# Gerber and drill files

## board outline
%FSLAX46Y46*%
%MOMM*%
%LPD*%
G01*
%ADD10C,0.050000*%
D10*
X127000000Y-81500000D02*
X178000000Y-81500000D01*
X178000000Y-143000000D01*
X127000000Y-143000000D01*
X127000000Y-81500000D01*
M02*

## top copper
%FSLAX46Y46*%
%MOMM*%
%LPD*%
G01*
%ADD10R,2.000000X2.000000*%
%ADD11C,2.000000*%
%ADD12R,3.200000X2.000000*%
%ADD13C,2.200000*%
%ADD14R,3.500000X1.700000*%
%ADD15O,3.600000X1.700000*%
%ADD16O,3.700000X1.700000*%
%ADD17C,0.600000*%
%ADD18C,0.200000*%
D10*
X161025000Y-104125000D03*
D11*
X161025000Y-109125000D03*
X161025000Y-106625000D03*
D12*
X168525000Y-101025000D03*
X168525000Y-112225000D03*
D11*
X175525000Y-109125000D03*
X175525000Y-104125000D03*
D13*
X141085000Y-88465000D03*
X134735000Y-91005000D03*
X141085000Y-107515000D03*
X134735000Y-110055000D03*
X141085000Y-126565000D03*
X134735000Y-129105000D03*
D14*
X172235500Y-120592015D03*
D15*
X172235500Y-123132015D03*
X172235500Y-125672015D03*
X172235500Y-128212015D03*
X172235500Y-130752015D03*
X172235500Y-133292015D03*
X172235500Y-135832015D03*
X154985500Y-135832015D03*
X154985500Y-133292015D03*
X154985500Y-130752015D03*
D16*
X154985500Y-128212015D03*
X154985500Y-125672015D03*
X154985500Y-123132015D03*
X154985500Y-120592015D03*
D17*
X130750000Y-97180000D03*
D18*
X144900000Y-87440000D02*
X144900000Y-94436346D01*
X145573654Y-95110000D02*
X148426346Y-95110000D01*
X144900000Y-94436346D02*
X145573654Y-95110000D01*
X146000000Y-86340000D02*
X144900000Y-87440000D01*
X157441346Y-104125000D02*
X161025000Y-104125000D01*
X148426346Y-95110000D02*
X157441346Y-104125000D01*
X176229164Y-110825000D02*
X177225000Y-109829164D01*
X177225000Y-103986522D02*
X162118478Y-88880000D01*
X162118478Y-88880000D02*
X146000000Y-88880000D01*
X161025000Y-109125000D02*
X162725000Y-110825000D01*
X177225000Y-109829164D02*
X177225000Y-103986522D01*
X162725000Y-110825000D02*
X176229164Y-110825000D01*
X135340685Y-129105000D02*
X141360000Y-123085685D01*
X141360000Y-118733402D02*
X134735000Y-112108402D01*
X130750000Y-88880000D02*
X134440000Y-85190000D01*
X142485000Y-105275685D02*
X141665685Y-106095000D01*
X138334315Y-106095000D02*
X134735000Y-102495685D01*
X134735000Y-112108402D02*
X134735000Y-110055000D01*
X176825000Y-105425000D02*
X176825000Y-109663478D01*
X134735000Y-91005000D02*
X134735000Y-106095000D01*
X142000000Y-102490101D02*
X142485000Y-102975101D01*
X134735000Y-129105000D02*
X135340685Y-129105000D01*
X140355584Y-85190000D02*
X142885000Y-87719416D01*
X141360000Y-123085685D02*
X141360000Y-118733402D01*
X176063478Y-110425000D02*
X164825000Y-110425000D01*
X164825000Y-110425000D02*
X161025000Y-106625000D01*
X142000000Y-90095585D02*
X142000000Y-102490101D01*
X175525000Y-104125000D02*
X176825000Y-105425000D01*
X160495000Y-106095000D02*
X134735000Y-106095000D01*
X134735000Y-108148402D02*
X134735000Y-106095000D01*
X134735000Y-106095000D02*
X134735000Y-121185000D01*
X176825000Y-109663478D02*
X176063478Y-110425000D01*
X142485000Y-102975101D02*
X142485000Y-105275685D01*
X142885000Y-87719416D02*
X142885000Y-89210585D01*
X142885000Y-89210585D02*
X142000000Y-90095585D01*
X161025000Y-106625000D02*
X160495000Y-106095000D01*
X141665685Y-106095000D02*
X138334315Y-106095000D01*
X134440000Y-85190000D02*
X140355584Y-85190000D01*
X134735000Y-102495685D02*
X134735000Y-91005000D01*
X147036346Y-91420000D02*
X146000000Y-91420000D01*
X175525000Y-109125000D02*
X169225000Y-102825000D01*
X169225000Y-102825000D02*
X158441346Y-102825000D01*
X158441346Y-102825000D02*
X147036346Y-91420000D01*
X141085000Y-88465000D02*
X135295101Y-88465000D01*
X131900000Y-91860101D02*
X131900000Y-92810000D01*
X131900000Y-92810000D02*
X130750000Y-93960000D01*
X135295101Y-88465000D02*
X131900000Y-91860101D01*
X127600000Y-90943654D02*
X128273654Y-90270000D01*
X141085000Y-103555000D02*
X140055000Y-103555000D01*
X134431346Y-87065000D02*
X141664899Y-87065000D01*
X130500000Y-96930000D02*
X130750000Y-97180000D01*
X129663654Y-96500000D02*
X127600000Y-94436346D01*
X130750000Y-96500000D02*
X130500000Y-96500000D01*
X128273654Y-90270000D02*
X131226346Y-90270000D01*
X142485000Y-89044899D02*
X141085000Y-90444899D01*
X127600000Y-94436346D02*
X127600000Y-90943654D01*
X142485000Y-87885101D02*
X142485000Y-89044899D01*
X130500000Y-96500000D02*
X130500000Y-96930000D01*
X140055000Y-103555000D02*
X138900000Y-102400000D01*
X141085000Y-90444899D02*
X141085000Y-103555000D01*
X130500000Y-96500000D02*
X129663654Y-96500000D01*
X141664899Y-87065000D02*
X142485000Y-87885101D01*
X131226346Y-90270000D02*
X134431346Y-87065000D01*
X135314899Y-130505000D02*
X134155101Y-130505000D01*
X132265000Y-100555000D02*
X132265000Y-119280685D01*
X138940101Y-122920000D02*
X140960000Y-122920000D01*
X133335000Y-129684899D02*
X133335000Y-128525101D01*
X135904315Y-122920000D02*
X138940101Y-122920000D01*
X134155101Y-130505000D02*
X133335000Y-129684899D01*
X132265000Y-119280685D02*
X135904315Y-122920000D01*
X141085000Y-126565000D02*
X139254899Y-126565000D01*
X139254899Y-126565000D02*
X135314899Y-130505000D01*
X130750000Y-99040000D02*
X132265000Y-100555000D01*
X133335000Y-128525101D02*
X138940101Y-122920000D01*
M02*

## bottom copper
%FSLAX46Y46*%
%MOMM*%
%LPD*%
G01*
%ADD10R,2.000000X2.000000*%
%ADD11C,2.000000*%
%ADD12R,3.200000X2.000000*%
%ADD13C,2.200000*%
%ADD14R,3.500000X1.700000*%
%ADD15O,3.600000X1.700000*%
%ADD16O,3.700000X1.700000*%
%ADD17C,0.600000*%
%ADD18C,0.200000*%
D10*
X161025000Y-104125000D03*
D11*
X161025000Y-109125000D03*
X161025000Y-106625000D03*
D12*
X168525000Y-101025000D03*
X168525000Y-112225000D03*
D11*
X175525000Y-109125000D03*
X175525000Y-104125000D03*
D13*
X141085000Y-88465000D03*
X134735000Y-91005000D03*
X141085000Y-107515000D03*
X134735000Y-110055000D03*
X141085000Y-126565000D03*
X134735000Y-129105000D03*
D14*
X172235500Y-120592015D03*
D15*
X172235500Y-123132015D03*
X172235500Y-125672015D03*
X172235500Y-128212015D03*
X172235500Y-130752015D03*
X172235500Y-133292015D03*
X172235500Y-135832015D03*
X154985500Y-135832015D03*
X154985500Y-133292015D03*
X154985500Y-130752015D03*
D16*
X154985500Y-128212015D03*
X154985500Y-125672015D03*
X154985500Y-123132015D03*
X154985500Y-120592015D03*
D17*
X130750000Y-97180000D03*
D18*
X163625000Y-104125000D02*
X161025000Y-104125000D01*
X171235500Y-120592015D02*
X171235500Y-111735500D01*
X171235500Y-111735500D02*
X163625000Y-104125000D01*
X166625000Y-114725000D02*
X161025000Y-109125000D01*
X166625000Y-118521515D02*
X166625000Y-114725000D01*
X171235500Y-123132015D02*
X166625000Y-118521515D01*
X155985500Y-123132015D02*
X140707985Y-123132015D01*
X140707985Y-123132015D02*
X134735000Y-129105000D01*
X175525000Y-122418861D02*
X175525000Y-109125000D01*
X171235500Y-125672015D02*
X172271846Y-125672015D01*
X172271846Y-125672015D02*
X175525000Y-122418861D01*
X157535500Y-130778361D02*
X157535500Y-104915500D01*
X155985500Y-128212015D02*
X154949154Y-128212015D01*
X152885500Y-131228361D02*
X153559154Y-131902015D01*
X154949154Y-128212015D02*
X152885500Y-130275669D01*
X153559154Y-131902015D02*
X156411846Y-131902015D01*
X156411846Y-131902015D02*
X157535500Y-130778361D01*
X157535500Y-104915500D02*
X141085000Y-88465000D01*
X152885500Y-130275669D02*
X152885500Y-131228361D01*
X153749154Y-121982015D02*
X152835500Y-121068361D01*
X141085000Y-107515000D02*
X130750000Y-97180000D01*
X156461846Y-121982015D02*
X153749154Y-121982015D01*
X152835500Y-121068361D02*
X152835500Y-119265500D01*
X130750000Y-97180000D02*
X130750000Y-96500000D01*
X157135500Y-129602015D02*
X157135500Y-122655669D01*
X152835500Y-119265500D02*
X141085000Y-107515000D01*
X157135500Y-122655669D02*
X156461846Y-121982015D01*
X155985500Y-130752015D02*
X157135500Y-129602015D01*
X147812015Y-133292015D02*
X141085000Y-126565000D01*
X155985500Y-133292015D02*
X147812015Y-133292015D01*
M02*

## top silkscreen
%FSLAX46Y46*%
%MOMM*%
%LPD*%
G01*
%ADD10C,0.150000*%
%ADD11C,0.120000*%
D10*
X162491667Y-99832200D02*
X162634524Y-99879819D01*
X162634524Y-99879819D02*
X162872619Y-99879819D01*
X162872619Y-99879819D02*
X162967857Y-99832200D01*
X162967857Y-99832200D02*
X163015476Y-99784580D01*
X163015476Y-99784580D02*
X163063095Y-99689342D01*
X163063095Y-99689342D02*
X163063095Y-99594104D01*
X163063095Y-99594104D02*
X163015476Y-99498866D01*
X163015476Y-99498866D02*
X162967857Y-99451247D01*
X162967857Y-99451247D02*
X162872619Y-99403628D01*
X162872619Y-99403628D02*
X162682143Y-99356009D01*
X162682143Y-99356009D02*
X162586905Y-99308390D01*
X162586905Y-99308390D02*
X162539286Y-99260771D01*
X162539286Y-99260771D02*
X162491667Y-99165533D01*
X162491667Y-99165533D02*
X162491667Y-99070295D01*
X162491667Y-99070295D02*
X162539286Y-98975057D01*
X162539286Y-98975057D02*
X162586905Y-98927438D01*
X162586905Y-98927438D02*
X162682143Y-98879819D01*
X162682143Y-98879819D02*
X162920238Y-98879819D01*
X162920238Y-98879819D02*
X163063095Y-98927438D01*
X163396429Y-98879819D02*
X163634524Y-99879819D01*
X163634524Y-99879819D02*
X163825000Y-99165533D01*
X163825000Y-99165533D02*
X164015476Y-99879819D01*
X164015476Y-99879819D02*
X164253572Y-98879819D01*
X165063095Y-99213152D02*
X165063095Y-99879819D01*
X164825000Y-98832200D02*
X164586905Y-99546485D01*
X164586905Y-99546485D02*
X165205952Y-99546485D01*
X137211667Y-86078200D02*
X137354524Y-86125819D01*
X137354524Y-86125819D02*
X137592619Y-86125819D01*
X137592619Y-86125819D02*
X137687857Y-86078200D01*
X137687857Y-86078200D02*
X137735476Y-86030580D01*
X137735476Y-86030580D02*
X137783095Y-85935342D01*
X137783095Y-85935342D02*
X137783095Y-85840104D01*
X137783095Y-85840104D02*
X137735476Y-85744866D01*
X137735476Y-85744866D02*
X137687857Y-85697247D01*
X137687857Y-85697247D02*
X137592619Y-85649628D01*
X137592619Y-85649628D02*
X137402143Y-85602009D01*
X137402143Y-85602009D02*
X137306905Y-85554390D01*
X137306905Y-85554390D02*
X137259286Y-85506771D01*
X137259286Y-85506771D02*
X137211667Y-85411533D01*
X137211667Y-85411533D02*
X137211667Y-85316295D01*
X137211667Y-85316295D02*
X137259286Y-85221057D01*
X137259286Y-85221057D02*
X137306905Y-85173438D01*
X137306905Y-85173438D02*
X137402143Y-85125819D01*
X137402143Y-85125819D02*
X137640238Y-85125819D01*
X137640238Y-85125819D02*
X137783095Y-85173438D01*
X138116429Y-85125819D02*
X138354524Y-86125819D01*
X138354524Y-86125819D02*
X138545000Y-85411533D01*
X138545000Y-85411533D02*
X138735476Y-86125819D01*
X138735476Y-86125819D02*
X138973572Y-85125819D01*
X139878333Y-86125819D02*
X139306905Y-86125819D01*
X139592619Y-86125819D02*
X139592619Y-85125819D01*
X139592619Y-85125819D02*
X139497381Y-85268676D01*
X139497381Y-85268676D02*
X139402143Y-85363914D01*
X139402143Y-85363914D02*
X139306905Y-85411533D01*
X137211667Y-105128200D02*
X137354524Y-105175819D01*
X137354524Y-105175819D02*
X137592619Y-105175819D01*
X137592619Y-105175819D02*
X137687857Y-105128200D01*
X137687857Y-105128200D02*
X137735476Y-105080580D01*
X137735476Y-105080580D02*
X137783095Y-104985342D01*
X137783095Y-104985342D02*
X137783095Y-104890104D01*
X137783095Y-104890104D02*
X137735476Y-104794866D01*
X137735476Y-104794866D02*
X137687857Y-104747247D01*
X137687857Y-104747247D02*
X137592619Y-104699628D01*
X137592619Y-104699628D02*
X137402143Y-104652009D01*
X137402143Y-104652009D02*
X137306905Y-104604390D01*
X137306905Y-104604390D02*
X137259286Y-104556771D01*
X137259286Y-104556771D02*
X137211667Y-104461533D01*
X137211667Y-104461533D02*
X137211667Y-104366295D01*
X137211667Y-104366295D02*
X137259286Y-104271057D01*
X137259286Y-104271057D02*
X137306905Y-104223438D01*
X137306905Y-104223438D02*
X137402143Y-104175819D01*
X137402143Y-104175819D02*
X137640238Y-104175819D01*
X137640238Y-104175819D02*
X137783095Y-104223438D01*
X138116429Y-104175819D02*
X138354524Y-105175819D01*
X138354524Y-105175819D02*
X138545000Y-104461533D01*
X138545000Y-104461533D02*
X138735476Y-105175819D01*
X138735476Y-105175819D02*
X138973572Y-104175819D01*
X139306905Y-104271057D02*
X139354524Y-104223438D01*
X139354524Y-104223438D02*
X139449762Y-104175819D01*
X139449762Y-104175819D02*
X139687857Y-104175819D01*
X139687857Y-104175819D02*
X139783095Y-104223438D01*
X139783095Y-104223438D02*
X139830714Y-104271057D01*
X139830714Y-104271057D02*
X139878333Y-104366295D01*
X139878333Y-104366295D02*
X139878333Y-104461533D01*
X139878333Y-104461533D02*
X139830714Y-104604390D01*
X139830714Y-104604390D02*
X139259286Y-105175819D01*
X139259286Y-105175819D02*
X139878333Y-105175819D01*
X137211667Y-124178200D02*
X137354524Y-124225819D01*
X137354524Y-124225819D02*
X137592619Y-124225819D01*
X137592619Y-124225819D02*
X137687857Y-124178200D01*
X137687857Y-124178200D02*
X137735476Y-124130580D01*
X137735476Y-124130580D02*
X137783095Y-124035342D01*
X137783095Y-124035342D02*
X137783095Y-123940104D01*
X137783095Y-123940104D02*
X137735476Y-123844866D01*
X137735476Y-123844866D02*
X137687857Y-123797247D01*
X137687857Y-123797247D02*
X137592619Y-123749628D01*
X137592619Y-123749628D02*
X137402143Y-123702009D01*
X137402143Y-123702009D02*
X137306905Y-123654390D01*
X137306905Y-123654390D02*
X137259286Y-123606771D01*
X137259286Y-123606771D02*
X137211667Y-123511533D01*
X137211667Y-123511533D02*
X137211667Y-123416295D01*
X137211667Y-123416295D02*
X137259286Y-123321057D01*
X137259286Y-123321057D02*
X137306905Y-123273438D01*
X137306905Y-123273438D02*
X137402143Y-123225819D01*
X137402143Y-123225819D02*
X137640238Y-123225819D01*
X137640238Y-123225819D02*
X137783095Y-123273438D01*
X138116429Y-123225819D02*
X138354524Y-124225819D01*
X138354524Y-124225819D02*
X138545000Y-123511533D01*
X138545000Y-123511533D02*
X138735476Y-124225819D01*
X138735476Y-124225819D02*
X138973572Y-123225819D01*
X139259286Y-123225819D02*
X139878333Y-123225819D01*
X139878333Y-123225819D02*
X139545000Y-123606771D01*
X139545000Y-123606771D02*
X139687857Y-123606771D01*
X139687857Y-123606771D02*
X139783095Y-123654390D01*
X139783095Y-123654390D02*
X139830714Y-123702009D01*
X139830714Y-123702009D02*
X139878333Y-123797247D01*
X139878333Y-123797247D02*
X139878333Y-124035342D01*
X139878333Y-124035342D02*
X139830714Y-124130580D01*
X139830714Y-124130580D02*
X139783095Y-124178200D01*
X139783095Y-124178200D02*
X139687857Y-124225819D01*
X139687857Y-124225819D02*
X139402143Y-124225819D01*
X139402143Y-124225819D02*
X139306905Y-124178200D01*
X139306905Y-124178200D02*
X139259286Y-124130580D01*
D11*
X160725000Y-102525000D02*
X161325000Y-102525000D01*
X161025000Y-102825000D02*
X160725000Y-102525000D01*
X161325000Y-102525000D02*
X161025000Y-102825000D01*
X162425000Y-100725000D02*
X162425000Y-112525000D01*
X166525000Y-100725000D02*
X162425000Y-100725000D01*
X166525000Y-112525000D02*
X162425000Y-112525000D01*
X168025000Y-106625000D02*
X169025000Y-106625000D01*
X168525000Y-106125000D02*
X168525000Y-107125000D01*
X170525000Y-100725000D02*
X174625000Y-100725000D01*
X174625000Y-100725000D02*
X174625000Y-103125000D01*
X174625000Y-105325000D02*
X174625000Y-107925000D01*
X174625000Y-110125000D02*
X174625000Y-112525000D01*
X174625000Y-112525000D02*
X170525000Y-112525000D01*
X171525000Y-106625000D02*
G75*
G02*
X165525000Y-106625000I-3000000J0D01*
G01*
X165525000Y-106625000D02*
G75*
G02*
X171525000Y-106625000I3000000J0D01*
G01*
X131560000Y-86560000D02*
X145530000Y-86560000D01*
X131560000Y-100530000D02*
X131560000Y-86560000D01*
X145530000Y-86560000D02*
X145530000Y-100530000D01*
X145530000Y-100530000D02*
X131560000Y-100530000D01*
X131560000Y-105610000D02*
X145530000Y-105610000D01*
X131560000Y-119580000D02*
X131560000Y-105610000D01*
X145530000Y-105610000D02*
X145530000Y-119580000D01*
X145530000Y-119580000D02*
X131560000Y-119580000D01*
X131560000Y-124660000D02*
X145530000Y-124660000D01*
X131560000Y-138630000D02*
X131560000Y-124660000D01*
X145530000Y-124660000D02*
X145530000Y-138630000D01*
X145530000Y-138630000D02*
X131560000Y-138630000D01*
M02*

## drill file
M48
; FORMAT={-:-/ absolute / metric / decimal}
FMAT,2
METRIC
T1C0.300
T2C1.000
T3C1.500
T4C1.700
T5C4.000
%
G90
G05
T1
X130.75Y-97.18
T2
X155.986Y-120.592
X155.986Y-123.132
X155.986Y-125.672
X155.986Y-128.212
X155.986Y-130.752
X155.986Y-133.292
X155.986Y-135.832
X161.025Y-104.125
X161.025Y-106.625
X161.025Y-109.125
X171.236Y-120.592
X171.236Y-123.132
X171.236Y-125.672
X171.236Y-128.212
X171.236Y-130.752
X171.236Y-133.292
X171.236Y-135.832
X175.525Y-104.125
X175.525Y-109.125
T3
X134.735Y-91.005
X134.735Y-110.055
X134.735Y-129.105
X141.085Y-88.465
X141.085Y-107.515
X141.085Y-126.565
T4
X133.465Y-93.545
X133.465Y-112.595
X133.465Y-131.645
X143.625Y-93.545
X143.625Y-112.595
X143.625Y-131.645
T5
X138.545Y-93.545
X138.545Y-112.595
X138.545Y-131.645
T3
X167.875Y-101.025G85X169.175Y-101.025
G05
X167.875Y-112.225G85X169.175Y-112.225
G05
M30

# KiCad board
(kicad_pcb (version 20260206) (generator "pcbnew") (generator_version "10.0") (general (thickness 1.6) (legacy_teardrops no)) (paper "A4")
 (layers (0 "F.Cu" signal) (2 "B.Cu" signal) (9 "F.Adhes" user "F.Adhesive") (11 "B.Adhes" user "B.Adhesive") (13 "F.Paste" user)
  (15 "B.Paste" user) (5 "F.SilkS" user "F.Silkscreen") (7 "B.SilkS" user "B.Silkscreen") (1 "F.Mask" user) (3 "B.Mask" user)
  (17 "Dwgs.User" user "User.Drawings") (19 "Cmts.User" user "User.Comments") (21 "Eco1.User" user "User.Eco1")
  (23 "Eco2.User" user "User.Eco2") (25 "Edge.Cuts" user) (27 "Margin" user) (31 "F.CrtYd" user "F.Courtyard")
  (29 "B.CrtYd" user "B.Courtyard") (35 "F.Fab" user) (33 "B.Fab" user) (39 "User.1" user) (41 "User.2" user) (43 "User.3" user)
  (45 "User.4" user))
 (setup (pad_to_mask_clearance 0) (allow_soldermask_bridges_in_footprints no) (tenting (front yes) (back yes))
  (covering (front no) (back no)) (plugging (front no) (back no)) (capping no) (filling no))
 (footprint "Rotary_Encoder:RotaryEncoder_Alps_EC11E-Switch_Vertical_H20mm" (layer "F.Cu") (at 161.025 104.125)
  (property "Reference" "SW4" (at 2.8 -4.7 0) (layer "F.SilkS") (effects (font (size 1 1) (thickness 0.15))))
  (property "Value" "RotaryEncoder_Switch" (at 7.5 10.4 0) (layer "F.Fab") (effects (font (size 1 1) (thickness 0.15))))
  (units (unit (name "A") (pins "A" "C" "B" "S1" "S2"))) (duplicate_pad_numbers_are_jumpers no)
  (fp_line (start -0.3 -1.6) (end 0.3 -1.6) (stroke (width 0.12) (type solid)) (layer "F.SilkS"))
  (fp_line (start 0 -1.3) (end -0.3 -1.6) (stroke (width 0.12) (type solid)) (layer "F.SilkS"))
  (fp_line (start 0.3 -1.6) (end 0 -1.3) (stroke (width 0.12) (type solid)) (layer "F.SilkS"))
  (fp_line (start 1.4 -3.4) (end 1.4 8.4) (stroke (width 0.12) (type solid)) (layer "F.SilkS"))
  (fp_line (start 5.5 -3.4) (end 1.4 -3.4) (stroke (width 0.12) (type solid)) (layer "F.SilkS"))
  (fp_line (start 5.5 8.4) (end 1.4 8.4) (stroke (width 0.12) (type solid)) (layer "F.SilkS"))
  (fp_line (start 7 2.5) (end 8 2.5) (stroke (width 0.12) (type solid)) (layer "F.SilkS"))
  (fp_line (start 7.5 2) (end 7.5 3) (stroke (width 0.12) (type solid)) (layer "F.SilkS"))
  (fp_line (start 9.5 -3.4) (end 13.6 -3.4) (stroke (width 0.12) (type solid)) (layer "F.SilkS"))
  (fp_line (start 13.6 -3.4) (end 13.6 -1) (stroke (width 0.12) (type solid)) (layer "F.SilkS"))
  (fp_line (start 13.6 1.2) (end 13.6 3.8) (stroke (width 0.12) (type solid)) (layer "F.SilkS"))
  (fp_line (start 13.6 6) (end 13.6 8.4) (stroke (width 0.12) (type solid)) (layer "F.SilkS"))
  (fp_line (start 13.6 8.4) (end 9.5 8.4) (stroke (width 0.12) (type solid)) (layer "F.SilkS"))
  (fp_circle (center 7.5 2.5) (end 10.5 2.5) (stroke (width 0.12) (type solid)) (fill no) (layer "F.SilkS"))
  (pad "A" thru_hole rect (at 0 0) (size 2 2) (drill 1) (layers "*.Cu" "*.Mask") (remove_unused_layers no) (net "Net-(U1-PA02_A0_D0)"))
  (pad "B" thru_hole circle (at 0 5) (size 2 2) (drill 1) (layers "*.Cu" "*.Mask") (remove_unused_layers no) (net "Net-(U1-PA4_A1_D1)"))
  (pad "C" thru_hole circle (at 0 2.5) (size 2 2) (drill 1) (layers "*.Cu" "*.Mask") (remove_unused_layers no) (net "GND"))
  (pad "MP" thru_hole rect (at 7.5 -3.1) (size 3.2 2) (drill oval 2.8 1.5) (layers "*.Cu" "*.Mask") (remove_unused_layers no))
  (pad "MP" thru_hole rect (at 7.5 8.1) (size 3.2 2) (drill oval 2.8 1.5) (layers "*.Cu" "*.Mask") (remove_unused_layers no))
  (pad "S1" thru_hole circle (at 14.5 5) (size 2 2) (drill 1) (layers "*.Cu" "*.Mask") (remove_unused_layers no) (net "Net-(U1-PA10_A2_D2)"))
  (pad "S2" thru_hole circle (at 14.5 0) (size 2 2) (drill 1) (layers "*.Cu" "*.Mask") (remove_unused_layers no) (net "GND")))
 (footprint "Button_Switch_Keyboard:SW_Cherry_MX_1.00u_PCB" (layer "F.Cu") (at 141.085 88.465)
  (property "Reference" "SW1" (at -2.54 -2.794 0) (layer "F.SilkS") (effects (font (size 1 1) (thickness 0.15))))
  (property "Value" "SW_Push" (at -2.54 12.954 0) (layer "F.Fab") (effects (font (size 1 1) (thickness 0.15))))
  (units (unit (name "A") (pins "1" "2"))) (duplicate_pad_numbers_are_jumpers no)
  (fp_line (start -9.525 -1.905) (end 4.445 -1.905) (stroke (width 0.12) (type solid)) (layer "F.SilkS"))
  (fp_line (start -9.525 12.065) (end -9.525 -1.905) (stroke (width 0.12) (type solid)) (layer "F.SilkS"))
  (fp_line (start 4.445 -1.905) (end 4.445 12.065) (stroke (width 0.12) (type solid)) (layer "F.SilkS"))
  (fp_line (start 4.445 12.065) (end -9.525 12.065) (stroke (width 0.12) (type solid)) (layer "F.SilkS"))
  (pad "" np_thru_hole circle (at -7.62 5.08) (size 1.7 1.7) (drill 1.7) (layers "*.Cu" "*.Mask"))
  (pad "" np_thru_hole circle (at -2.54 5.08) (size 4 4) (drill 4) (layers "*.Cu" "*.Mask"))
  (pad "" np_thru_hole circle (at 2.54 5.08) (size 1.7 1.7) (drill 1.7) (layers "*.Cu" "*.Mask"))
  (pad "1" thru_hole circle (at 0 0) (size 2.2 2.2) (drill 1.5) (layers "*.Cu" "*.Mask") (remove_unused_layers no)
   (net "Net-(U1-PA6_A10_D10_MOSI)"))
  (pad "2" thru_hole circle (at -6.35 2.54) (size 2.2 2.2) (drill 1.5) (layers "*.Cu" "*.Mask") (remove_unused_layers no) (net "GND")))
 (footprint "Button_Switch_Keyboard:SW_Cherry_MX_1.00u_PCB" (layer "F.Cu") (at 141.085 107.515)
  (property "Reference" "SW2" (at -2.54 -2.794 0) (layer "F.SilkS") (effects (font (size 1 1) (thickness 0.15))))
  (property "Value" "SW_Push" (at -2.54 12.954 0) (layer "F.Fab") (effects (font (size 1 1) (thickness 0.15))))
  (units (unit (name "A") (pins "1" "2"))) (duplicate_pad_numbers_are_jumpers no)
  (fp_line (start -9.525 -1.905) (end 4.445 -1.905) (stroke (width 0.12) (type solid)) (layer "F.SilkS"))
  (fp_line (start -9.525 12.065) (end -9.525 -1.905) (stroke (width 0.12) (type solid)) (layer "F.SilkS"))
  (fp_line (start 4.445 -1.905) (end 4.445 12.065) (stroke (width 0.12) (type solid)) (layer "F.SilkS"))
  (fp_line (start 4.445 12.065) (end -9.525 12.065) (stroke (width 0.12) (type solid)) (layer "F.SilkS"))
  (pad "" np_thru_hole circle (at -7.62 5.08) (size 1.7 1.7) (drill 1.7) (layers "*.Cu" "*.Mask"))
  (pad "" np_thru_hole circle (at -2.54 5.08) (size 4 4) (drill 4) (layers "*.Cu" "*.Mask"))
  (pad "" np_thru_hole circle (at 2.54 5.08) (size 1.7 1.7) (drill 1.7) (layers "*.Cu" "*.Mask"))
  (pad "1" thru_hole circle (at 0 0) (size 2.2 2.2) (drill 1.5) (layers "*.Cu" "*.Mask") (remove_unused_layers no)
   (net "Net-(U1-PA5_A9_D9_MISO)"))
  (pad "2" thru_hole circle (at -6.35 2.54) (size 2.2 2.2) (drill 1.5) (layers "*.Cu" "*.Mask") (remove_unused_layers no) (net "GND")))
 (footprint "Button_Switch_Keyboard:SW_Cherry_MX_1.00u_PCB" (layer "F.Cu") (at 141.085 126.565)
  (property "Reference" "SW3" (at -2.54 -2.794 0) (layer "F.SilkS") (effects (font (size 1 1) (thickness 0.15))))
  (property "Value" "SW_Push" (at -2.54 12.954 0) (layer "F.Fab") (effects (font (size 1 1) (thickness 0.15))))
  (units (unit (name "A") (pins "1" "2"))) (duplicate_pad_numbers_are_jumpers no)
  (fp_line (start -9.525 -1.905) (end 4.445 -1.905) (stroke (width 0.12) (type solid)) (layer "F.SilkS"))
  (fp_line (start -9.525 12.065) (end -9.525 -1.905) (stroke (width 0.12) (type solid)) (layer "F.SilkS"))
  (fp_line (start 4.445 -1.905) (end 4.445 12.065) (stroke (width 0.12) (type solid)) (layer "F.SilkS"))
  (fp_line (start 4.445 12.065) (end -9.525 12.065) (stroke (width 0.12) (type solid)) (layer "F.SilkS"))
  (pad "" np_thru_hole circle (at -7.62 5.08) (size 1.7 1.7) (drill 1.7) (layers "*.Cu" "*.Mask"))
  (pad "" np_thru_hole circle (at -2.54 5.08) (size 4 4) (drill 4) (layers "*.Cu" "*.Mask"))
  (pad "" np_thru_hole circle (at 2.54 5.08) (size 1.7 1.7) (drill 1.7) (layers "*.Cu" "*.Mask"))
  (pad "1" thru_hole circle (at 0 0) (size 2.2 2.2) (drill 1.5) (layers "*.Cu" "*.Mask") (remove_unused_layers no)
   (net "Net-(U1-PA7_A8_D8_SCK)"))
  (pad "2" thru_hole circle (at -6.35 2.54) (size 2.2 2.2) (drill 1.5) (layers "*.Cu" "*.Mask") (remove_unused_layers no) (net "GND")))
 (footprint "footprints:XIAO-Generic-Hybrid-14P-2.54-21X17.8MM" (layer "B.Cu") (at 163.6105 128.212015 180)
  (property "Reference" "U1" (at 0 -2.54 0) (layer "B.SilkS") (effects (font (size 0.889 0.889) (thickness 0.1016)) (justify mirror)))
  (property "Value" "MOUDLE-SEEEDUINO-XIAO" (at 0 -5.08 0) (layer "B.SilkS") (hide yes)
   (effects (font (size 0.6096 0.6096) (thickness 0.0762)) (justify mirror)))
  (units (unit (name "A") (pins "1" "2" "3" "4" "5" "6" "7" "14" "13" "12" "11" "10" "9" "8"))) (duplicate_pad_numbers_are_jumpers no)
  (pad "1" thru_hole rect (at -7.625 7.62 180) (size 3.5 1.7) (drill 1 (offset -1 0)) (layers "*.Cu" "*.Mask") (remove_unused_layers no)
   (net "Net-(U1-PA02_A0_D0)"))
  (pad "2" thru_hole oval (at -7.625 5.08 180) (size 3.6 1.7) (drill 1 (offset -1 0)) (layers "*.Cu" "*.Mask") (remove_unused_layers no)
   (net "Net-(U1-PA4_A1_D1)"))
  (pad "3" thru_hole oval (at -7.625 2.54 180) (size 3.6 1.7) (drill 1 (offset -1 0)) (layers "*.Cu" "*.Mask") (remove_unused_layers no)
   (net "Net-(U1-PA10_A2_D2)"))
  (pad "4" thru_hole oval (at -7.625 0 180) (size 3.6 1.7) (drill 1 (offset -1 0)) (layers "*.Cu" "*.Mask") (remove_unused_layers no)
   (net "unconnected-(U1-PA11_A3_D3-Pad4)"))
  (pad "5" thru_hole oval (at -7.625 -2.54 180) (size 3.6 1.7) (drill 1 (offset -1 0)) (layers "*.Cu" "*.Mask") (remove_unused_layers no)
   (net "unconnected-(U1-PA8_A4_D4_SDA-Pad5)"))
  (pad "6" thru_hole oval (at -7.625 -5.08) (size 3.6 1.7) (drill 1 (offset 1 0)) (layers "*.Cu" "*.Mask") (remove_unused_layers no)
   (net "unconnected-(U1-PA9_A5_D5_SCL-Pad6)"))
  (pad "7" thru_hole oval (at -7.625 -7.62 180) (size 3.6 1.7) (drill 1 (offset -1 0)) (layers "*.Cu" "*.Mask") (remove_unused_layers no)
   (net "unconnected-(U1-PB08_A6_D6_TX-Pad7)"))
  (pad "8" thru_hole oval (at 7.625 -7.62 180) (size 3.6 1.7) (drill 1 (offset 1 0)) (layers "*.Cu" "*.Mask") (remove_unused_layers no)
   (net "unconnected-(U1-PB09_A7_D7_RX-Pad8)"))
  (pad "9" thru_hole oval (at 7.625 -5.08 180) (size 3.6 1.7) (drill 1 (offset 1 0)) (layers "*.Cu" "*.Mask") (remove_unused_layers no)
   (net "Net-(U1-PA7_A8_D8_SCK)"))
  (pad "10" thru_hole oval (at 7.625 -2.54 180) (size 3.6 1.7) (drill 1 (offset 1 0)) (layers "*.Cu" "*.Mask") (remove_unused_layers no)
   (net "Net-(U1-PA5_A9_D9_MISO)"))
  (pad "11" thru_hole oval (at 7.625 0 180) (size 3.7 1.7) (drill 1 (offset 1 0)) (layers "*.Cu" "*.Mask") (remove_unused_layers no)
   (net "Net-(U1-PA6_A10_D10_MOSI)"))
  (pad "12" thru_hole oval (at 7.625 2.54 180) (size 3.7 1.7) (drill 1 (offset 1 0)) (layers "*.Cu" "*.Mask") (remove_unused_layers no)
   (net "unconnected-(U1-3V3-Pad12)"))
  (pad "13" thru_hole oval (at 7.625 5.08 180) (size 3.7 1.7) (drill 1 (offset 1 0)) (layers "*.Cu" "*.Mask") (remove_unused_layers no)
   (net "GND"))
  (pad "14" thru_hole oval (at 7.625 7.62 180) (size 3.7 1.7) (drill 1 (offset 1 0)) (layers "*.Cu" "*.Mask") (remove_unused_layers no)
   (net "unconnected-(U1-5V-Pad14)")))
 (gr_rect (start 127 81.5) (end 178 143) (stroke (width 0.05) (type solid)) (fill no) (layer "Edge.Cuts"))
 (segment (start 144.9 87.44) (end 144.9 94.436346) (width 0.2) (layer "F.Cu") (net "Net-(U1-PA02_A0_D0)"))
 (segment (start 145.573654 95.11) (end 148.426346 95.11) (width 0.2) (layer "F.Cu") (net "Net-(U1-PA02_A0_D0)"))
 (segment (start 144.9 94.436346) (end 145.573654 95.11) (width 0.2) (layer "F.Cu") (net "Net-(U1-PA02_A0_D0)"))
 (segment (start 146 86.34) (end 144.9 87.44) (width 0.2) (layer "F.Cu") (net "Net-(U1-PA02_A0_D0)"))
 (segment (start 157.441346 104.125) (end 161.025 104.125) (width 0.2) (layer "F.Cu") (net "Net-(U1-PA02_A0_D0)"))
 (segment (start 148.426346 95.11) (end 157.441346 104.125) (width 0.2) (layer "F.Cu") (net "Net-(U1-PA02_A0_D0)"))
 (segment (start 163.625 104.125) (end 161.025 104.125) (width 0.2) (layer "B.Cu") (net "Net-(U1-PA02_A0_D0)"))
 (segment (start 171.2355 120.592015) (end 171.2355 111.7355) (width 0.2) (layer "B.Cu") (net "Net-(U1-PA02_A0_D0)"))
 (segment (start 171.2355 111.7355) (end 163.625 104.125) (width 0.2) (layer "B.Cu") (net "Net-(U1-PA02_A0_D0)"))
 (segment (start 176.229164 110.825) (end 177.225 109.829164) (width 0.2) (layer "F.Cu") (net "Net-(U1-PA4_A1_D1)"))
 (segment (start 177.225 103.986522) (end 162.118478 88.88) (width 0.2) (layer "F.Cu") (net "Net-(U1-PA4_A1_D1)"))
 (segment (start 162.118478 88.88) (end 146 88.88) (width 0.2) (layer "F.Cu") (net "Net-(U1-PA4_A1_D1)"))
 (segment (start 161.025 109.125) (end 162.725 110.825) (width 0.2) (layer "F.Cu") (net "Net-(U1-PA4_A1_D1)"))
 (segment (start 177.225 109.829164) (end 177.225 103.986522) (width 0.2) (layer "F.Cu") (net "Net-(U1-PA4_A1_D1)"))
 (segment (start 162.725 110.825) (end 176.229164 110.825) (width 0.2) (layer "F.Cu") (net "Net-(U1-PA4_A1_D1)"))
 (segment (start 166.625 114.725) (end 161.025 109.125) (width 0.2) (layer "B.Cu") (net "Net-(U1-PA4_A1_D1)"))
 (segment (start 166.625 118.521515) (end 166.625 114.725) (width 0.2) (layer "B.Cu") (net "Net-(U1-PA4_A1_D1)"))
 (segment (start 171.2355 123.132015) (end 166.625 118.521515) (width 0.2) (layer "B.Cu") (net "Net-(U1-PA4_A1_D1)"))
 (segment (start 135.340685 129.105) (end 141.36 123.085685) (width 0.2) (layer "F.Cu") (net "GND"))
 (segment (start 141.36 118.733402) (end 134.735 112.108402) (width 0.2) (layer "F.Cu") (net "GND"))
 (segment (start 130.75 88.88) (end 134.44 85.19) (width 0.2) (layer "F.Cu") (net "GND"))
 (segment (start 142.485 105.275685) (end 141.665685 106.095) (width 0.2) (layer "F.Cu") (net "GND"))
 (segment (start 138.334315 106.095) (end 134.735 102.495685) (width 0.2) (layer "F.Cu") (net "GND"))
 (segment (start 134.735 112.108402) (end 134.735 110.055) (width 0.2) (layer "F.Cu") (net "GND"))
 (segment (start 176.825 105.425) (end 176.825 109.663478) (width 0.2) (layer "F.Cu") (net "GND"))
 (segment (start 134.735 91.005) (end 134.735 106.095) (width 0.2) (layer "F.Cu") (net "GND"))
 (segment (start 142 102.490101) (end 142.485 102.975101) (width 0.2) (layer "F.Cu") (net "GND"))
 (segment (start 134.735 129.105) (end 135.340685 129.105) (width 0.2) (layer "F.Cu") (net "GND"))
 (segment (start 140.355584 85.19) (end 142.885 87.719416) (width 0.2) (layer "F.Cu") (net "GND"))
 (segment (start 141.36 123.085685) (end 141.36 118.733402) (width 0.2) (layer "F.Cu") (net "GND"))
 (segment (start 176.063478 110.425) (end 164.825 110.425) (width 0.2) (layer "F.Cu") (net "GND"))
 (segment (start 164.825 110.425) (end 161.025 106.625) (width 0.2) (layer "F.Cu") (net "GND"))
 (segment (start 142 90.095585) (end 142 102.490101) (width 0.2) (layer "F.Cu") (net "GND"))
 (segment (start 175.525 104.125) (end 176.825 105.425) (width 0.2) (layer "F.Cu") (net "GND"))
 (segment (start 160.495 106.095) (end 134.735 106.095) (width 0.2) (layer "F.Cu") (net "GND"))
 (segment (start 134.735 108.148402) (end 134.735 106.095) (width 0.2) (layer "F.Cu") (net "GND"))
 (segment (start 134.735 106.095) (end 134.735 121.185) (width 0.2) (layer "F.Cu") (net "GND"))
 (segment (start 176.825 109.663478) (end 176.063478 110.425) (width 0.2) (layer "F.Cu") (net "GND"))
 (segment (start 142.485 102.975101) (end 142.485 105.275685) (width 0.2) (layer "F.Cu") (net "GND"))
 (segment (start 142.885 87.719416) (end 142.885 89.210585) (width 0.2) (layer "F.Cu") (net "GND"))
 (segment (start 142.885 89.210585) (end 142 90.095585) (width 0.2) (layer "F.Cu") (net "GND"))
 (segment (start 161.025 106.625) (end 160.495 106.095) (width 0.2) (layer "F.Cu") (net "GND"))
 (segment (start 141.665685 106.095) (end 138.334315 106.095) (width 0.2) (layer "F.Cu") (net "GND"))
 (segment (start 134.44 85.19) (end 140.355584 85.19) (width 0.2) (layer "F.Cu") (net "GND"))
 (segment (start 134.735 102.495685) (end 134.735 91.005) (width 0.2) (layer "F.Cu") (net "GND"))
 (segment (start 155.9855 123.132015) (end 140.707985 123.132015) (width 0.2) (layer "B.Cu") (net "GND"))
 (segment (start 140.707985 123.132015) (end 134.735 129.105) (width 0.2) (layer "B.Cu") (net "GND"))
 (segment (start 147.036346 91.42) (end 146 91.42) (width 0.2) (layer "F.Cu") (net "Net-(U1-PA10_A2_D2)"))
 (segment (start 175.525 109.125) (end 169.225 102.825) (width 0.2) (layer "F.Cu") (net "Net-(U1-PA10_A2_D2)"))
 (segment (start 169.225 102.825) (end 158.441346 102.825) (width 0.2) (layer "F.Cu") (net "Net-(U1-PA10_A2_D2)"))
 (segment (start 158.441346 102.825) (end 147.036346 91.42) (width 0.2) (layer "F.Cu") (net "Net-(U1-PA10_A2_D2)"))
 (segment (start 175.525 122.418861) (end 175.525 109.125) (width 0.2) (layer "B.Cu") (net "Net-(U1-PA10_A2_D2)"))
 (segment (start 171.2355 125.672015) (end 172.271846 125.672015) (width 0.2) (layer "B.Cu") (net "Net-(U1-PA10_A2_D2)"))
 (segment (start 172.271846 125.672015) (end 175.525 122.418861) (width 0.2) (layer "B.Cu") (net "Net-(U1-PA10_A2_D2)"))
 (segment (start 141.085 88.465) (end 135.295101 88.465) (width 0.2) (layer "F.Cu") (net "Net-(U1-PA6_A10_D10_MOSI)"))
 (segment (start 131.9 91.860101) (end 131.9 92.81) (width 0.2) (layer "F.Cu") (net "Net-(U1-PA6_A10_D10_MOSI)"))
 (segment (start 131.9 92.81) (end 130.75 93.96) (width 0.2) (layer "F.Cu") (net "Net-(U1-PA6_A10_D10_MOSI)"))
 (segment (start 135.295101 88.465) (end 131.9 91.860101) (width 0.2) (layer "F.Cu") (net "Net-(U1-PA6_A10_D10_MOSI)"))
 (segment (start 157.5355 130.778361) (end 157.5355 104.9155) (width 0.2) (layer "B.Cu") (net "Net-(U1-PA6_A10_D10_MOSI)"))
 (segment (start 155.9855 128.212015) (end 154.949154 128.212015) (width 0.2) (layer "B.Cu") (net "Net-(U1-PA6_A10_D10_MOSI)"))
 (segment (start 152.8855 131.228361) (end 153.559154 131.902015) (width 0.2) (layer "B.Cu") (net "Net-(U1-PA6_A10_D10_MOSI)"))
 (segment (start 154.949154 128.212015) (end 152.8855 130.275669) (width 0.2) (layer "B.Cu") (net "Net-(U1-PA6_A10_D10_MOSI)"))
 (segment (start 153.559154 131.902015) (end 156.411846 131.902015) (width 0.2) (layer "B.Cu") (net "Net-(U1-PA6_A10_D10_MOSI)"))
 (segment (start 156.411846 131.902015) (end 157.5355 130.778361) (width 0.2) (layer "B.Cu") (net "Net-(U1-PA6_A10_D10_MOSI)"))
 (segment (start 157.5355 104.9155) (end 141.085 88.465) (width 0.2) (layer "B.Cu") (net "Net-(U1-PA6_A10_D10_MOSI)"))
 (segment (start 152.8855 130.275669) (end 152.8855 131.228361) (width 0.2) (layer "B.Cu") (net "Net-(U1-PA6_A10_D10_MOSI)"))
 (segment (start 127.6 90.943654) (end 128.273654 90.27) (width 0.2) (layer "F.Cu") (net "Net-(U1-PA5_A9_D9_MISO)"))
 (segment (start 141.085 103.555) (end 140.055 103.555) (width 0.2) (layer "F.Cu") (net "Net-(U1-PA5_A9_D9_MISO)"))
 (segment (start 134.431346 87.065) (end 141.664899 87.065) (width 0.2) (layer "F.Cu") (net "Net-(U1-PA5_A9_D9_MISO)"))
 (segment (start 130.5 96.93) (end 130.75 97.18) (width 0.2) (layer "F.Cu") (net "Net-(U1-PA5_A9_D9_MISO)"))
 (segment (start 129.663654 96.5) (end 127.6 94.436346) (width 0.2) (layer "F.Cu") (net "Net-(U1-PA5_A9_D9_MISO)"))
 (segment (start 130.75 96.5) (end 130.5 96.5) (width 0.2) (layer "F.Cu") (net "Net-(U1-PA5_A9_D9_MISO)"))
 (segment (start 128.273654 90.27) (end 131.226346 90.27) (width 0.2) (layer "F.Cu") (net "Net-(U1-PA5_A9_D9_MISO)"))
 (segment (start 142.485 89.044899) (end 141.085 90.444899) (width 0.2) (layer "F.Cu") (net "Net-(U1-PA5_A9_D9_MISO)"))
 (segment (start 127.6 94.436346) (end 127.6 90.943654) (width 0.2) (layer "F.Cu") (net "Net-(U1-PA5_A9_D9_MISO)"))
 (segment (start 142.485 87.885101) (end 142.485 89.044899) (width 0.2) (layer "F.Cu") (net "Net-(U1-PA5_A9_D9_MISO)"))
 (segment (start 130.5 96.5) (end 130.5 96.93) (width 0.2) (layer "F.Cu") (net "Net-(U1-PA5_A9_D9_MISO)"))
 (segment (start 140.055 103.555) (end 138.9 102.4) (width 0.2) (layer "F.Cu") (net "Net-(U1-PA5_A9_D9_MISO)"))
 (segment (start 141.085 90.444899) (end 141.085 103.555) (width 0.2) (layer "F.Cu") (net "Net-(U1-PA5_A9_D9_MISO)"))
 (segment (start 130.5 96.5) (end 129.663654 96.5) (width 0.2) (layer "F.Cu") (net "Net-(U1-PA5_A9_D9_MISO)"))
 (segment (start 141.664899 87.065) (end 142.485 87.885101) (width 0.2) (layer "F.Cu") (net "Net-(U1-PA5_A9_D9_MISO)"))
 (segment (start 131.226346 90.27) (end 134.431346 87.065) (width 0.2) (layer "F.Cu") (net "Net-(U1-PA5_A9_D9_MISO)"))
 (via (at 130.75 97.18) (size 0.6) (drill 0.3) (layers "F.Cu" "B.Cu") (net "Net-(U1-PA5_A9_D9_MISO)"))
 (segment (start 153.749154 121.982015) (end 152.8355 121.068361) (width 0.2) (layer "B.Cu") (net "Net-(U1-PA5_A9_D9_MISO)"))
 (segment (start 141.085 107.515) (end 130.75 97.18) (width 0.2) (layer "B.Cu") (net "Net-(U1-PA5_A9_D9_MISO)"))
 (segment (start 156.461846 121.982015) (end 153.749154 121.982015) (width 0.2) (layer "B.Cu") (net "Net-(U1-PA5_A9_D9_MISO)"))
 (segment (start 152.8355 121.068361) (end 152.8355 119.2655) (width 0.2) (layer "B.Cu") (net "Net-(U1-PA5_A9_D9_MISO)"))
 (segment (start 130.75 97.18) (end 130.75 96.5) (width 0.2) (layer "B.Cu") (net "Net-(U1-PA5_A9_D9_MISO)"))
 (segment (start 157.1355 129.602015) (end 157.1355 122.655669) (width 0.2) (layer "B.Cu") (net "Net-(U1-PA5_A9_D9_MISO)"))
 (segment (start 152.8355 119.2655) (end 141.085 107.515) (width 0.2) (layer "B.Cu") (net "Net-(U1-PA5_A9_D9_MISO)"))
 (segment (start 157.1355 122.655669) (end 156.461846 121.982015) (width 0.2) (layer "B.Cu") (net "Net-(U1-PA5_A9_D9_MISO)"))
 (segment (start 155.9855 130.752015) (end 157.1355 129.602015) (width 0.2) (layer "B.Cu") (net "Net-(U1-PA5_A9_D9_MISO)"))
 (segment (start 135.314899 130.505) (end 134.155101 130.505) (width 0.2) (layer "F.Cu") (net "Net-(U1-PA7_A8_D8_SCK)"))
 (segment (start 132.265 100.555) (end 132.265 119.280685) (width 0.2) (layer "F.Cu") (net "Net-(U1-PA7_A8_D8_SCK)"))
 (segment (start 138.940101 122.92) (end 140.96 122.92) (width 0.2) (layer "F.Cu") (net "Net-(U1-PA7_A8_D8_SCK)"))
 (segment (start 133.335 129.684899) (end 133.335 128.525101) (width 0.2) (layer "F.Cu") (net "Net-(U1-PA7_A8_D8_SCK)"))
 (segment (start 135.904315 122.92) (end 138.940101 122.92) (width 0.2) (layer "F.Cu") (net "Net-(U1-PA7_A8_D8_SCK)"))
 (segment (start 134.155101 130.505) (end 133.335 129.684899) (width 0.2) (layer "F.Cu") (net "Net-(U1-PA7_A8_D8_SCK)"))
 (segment (start 132.265 119.280685) (end 135.904315 122.92) (width 0.2) (layer "F.Cu") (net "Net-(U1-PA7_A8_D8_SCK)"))
 (segment (start 141.085 126.565) (end 139.254899 126.565) (width 0.2) (layer "F.Cu") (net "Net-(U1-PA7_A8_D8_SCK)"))
 (segment (start 139.254899 126.565) (end 135.314899 130.505) (width 0.2) (layer "F.Cu") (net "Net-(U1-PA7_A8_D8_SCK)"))
 (segment (start 130.75 99.04) (end 132.265 100.555) (width 0.2) (layer "F.Cu") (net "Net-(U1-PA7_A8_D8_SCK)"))
 (segment (start 133.335 128.525101) (end 138.940101 122.92) (width 0.2) (layer "F.Cu") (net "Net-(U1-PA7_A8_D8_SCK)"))
 (segment (start 147.812015 133.292015) (end 141.085 126.565) (width 0.2) (layer "B.Cu") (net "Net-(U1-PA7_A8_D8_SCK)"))
 (segment (start 155.9855 133.292015) (end 147.812015 133.292015) (width 0.2) (layer "B.Cu") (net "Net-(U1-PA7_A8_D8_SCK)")))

